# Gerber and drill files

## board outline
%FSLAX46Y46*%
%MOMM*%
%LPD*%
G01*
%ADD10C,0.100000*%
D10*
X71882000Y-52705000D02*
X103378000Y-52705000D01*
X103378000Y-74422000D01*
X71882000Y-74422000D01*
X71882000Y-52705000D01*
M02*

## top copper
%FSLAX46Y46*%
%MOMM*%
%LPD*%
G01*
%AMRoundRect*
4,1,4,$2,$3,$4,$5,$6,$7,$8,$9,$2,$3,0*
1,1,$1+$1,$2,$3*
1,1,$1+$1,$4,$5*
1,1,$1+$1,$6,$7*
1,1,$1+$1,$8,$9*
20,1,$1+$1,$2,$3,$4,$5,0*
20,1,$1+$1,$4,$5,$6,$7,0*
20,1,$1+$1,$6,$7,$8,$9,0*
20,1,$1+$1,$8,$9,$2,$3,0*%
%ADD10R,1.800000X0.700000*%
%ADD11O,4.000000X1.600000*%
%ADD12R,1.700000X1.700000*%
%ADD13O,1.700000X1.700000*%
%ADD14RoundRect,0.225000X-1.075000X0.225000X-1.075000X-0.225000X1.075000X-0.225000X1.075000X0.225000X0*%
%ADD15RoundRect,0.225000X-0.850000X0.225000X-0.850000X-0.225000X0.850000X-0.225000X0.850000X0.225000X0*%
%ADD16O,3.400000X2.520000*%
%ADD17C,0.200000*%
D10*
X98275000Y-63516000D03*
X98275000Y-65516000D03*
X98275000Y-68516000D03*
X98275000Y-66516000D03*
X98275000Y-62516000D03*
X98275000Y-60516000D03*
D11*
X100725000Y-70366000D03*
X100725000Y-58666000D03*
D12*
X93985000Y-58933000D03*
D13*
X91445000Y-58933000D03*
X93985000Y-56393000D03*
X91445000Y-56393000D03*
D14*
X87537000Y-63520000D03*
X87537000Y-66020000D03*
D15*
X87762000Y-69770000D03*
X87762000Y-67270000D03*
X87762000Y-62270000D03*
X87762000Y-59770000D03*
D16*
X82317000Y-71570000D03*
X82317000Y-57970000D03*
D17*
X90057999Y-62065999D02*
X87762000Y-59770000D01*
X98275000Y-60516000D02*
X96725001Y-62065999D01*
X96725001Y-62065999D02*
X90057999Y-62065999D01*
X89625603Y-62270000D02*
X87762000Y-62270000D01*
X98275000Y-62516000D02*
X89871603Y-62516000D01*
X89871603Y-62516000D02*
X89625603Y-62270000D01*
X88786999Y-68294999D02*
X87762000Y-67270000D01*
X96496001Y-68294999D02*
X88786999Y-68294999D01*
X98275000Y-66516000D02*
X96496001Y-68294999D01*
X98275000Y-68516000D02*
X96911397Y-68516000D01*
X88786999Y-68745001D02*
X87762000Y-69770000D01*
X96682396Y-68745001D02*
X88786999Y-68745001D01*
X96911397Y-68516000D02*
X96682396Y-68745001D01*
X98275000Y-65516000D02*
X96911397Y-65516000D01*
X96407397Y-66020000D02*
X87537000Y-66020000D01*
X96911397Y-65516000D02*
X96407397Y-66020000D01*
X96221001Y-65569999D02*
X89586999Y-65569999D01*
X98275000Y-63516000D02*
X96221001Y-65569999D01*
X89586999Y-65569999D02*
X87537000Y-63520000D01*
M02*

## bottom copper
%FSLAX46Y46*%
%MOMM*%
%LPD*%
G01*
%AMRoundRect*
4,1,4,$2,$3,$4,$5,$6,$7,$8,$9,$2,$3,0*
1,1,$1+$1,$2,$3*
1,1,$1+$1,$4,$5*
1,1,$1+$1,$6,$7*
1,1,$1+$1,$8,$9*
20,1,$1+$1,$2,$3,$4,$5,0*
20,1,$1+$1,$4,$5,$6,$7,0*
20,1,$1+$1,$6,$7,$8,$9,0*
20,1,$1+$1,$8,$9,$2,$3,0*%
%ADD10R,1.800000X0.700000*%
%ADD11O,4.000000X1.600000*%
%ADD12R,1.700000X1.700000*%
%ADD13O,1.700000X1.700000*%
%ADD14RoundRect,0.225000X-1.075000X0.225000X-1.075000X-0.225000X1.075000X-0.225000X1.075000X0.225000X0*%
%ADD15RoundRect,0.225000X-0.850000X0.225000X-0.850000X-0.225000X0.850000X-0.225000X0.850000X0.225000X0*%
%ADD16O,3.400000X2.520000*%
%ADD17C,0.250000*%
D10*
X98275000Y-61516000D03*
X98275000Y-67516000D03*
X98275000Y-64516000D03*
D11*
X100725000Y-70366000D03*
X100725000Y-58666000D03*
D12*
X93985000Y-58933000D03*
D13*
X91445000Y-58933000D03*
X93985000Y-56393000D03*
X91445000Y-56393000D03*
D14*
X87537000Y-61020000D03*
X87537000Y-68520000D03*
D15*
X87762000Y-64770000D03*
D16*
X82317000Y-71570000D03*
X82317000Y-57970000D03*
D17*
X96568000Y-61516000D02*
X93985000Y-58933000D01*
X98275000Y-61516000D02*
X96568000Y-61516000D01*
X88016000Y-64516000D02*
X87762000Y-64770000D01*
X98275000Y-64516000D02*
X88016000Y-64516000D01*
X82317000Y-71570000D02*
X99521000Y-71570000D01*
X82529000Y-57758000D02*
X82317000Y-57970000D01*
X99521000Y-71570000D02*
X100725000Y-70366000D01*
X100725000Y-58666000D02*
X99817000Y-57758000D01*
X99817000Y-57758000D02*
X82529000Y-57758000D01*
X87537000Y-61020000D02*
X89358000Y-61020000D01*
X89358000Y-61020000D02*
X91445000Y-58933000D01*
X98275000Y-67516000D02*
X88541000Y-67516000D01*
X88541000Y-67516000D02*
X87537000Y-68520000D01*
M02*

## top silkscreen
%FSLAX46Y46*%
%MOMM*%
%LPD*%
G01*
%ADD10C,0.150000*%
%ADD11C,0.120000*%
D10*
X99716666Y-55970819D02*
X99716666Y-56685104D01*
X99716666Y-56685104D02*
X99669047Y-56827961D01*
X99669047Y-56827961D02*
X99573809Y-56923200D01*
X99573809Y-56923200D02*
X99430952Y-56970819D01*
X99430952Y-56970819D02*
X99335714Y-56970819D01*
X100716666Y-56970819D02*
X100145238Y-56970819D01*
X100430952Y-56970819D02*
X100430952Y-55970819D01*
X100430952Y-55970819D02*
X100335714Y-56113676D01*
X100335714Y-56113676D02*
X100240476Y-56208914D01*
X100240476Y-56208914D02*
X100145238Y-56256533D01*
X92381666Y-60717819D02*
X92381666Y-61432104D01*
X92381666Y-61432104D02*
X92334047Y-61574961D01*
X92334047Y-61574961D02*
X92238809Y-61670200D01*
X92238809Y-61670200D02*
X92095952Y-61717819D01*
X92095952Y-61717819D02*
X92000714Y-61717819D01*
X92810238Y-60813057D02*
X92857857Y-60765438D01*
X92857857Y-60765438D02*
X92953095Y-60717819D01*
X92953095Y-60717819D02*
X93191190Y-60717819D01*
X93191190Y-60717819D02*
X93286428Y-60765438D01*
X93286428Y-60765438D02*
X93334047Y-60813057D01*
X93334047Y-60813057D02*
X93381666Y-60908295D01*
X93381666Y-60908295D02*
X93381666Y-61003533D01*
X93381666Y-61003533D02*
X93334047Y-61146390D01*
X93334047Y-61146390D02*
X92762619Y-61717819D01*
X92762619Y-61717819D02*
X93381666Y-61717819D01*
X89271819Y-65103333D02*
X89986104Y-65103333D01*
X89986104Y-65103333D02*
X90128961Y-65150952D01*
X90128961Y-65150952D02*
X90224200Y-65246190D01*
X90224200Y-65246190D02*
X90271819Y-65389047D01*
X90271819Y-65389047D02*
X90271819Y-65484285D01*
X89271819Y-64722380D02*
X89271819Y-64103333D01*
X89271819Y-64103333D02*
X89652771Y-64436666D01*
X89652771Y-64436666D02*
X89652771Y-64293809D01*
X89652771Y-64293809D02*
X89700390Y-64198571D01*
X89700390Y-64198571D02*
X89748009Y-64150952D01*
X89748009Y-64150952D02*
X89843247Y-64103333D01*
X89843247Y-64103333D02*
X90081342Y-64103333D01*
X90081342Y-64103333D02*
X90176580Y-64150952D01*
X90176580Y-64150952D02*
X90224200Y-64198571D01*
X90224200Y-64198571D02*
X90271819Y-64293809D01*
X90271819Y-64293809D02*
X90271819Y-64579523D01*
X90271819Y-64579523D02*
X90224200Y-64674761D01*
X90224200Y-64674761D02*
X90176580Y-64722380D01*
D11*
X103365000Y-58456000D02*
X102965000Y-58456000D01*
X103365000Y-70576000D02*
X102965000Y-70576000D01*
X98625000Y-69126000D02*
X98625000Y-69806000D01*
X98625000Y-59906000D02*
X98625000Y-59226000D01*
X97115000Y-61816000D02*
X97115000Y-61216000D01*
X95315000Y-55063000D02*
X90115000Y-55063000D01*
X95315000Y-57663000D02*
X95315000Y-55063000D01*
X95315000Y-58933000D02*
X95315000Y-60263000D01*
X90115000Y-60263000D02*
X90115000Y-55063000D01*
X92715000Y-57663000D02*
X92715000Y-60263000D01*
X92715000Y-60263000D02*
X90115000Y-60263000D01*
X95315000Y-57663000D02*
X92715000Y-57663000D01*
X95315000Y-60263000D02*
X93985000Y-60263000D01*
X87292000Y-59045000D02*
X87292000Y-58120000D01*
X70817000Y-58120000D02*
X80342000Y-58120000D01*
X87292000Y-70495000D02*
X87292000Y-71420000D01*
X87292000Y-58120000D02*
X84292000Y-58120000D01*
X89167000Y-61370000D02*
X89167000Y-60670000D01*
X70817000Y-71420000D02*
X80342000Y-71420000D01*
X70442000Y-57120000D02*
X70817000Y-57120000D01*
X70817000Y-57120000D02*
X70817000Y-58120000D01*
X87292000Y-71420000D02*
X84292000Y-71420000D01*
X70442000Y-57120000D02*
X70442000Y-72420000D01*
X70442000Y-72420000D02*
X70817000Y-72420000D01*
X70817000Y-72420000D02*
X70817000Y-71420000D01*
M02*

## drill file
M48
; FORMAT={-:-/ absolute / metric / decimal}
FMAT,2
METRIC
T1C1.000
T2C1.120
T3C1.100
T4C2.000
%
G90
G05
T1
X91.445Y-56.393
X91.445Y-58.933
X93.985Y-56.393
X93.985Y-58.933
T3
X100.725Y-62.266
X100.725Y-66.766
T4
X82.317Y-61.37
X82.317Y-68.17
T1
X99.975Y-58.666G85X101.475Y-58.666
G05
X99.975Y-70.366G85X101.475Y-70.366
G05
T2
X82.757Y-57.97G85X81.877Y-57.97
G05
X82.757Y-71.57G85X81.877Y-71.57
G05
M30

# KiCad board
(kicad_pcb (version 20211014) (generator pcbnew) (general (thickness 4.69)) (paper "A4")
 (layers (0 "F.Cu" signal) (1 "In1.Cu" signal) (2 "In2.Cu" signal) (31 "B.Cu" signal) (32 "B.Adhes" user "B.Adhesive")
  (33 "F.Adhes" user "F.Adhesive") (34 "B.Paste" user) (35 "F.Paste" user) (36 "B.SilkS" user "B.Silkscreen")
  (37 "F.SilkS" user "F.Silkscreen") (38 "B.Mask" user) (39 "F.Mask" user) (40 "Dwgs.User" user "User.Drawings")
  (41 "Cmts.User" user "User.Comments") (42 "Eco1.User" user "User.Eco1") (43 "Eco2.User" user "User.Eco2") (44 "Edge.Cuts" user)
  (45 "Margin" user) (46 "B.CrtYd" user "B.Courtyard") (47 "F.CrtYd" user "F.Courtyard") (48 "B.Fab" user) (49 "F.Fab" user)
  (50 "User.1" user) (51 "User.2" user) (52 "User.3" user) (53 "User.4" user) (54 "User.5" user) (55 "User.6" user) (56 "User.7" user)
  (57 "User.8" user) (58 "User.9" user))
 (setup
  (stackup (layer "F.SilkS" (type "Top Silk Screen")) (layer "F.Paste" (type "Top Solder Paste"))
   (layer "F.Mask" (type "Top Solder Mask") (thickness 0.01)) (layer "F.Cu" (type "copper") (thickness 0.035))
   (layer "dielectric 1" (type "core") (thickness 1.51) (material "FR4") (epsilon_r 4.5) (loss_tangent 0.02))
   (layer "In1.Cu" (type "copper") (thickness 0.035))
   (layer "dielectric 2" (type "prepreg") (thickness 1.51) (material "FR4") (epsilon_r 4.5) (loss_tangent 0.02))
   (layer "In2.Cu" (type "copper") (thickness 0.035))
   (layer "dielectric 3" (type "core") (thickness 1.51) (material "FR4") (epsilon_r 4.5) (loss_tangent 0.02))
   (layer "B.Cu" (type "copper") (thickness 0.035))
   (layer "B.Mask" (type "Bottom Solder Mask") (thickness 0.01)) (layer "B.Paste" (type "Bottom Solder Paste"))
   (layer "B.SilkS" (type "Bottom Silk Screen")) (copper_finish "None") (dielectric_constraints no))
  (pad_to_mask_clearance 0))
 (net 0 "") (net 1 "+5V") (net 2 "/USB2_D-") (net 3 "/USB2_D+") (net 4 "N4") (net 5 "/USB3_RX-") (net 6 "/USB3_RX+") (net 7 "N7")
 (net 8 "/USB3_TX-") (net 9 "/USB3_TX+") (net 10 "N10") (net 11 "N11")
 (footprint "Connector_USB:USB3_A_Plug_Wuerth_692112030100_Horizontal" (layer "F.Cu") (at 100.05 64.516)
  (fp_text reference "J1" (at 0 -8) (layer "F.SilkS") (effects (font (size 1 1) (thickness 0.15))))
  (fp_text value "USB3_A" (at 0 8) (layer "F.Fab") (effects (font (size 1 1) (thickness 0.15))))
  (fp_line (start 3.315 -6.06) (end 2.915 -6.06) (layer "F.SilkS") (width 0.12))
  (fp_line (start 3.315 6.06) (end 2.915 6.06) (layer "F.SilkS") (width 0.12))
  (fp_line (start -1.425 4.61) (end -1.425 5.29) (layer "F.SilkS") (width 0.12))
  (fp_line (start -1.425 -4.61) (end -1.425 -5.29) (layer "F.SilkS") (width 0.12))
  (fp_line (start -2.935 -2.7) (end -2.935 -3.3) (layer "F.SilkS") (width 0.12))
  (pad "" np_thru_hole circle (at 0.675 2.25 90) (size 1.1 1.1) (drill 1.1) (layers *.Cu *.Mask))
  (pad "" np_thru_hole circle (at 0.675 -2.25 90) (size 1.1 1.1) (drill 1.1) (layers *.Cu *.Mask))
  (pad "1" smd rect (at -1.775 -3 90) (size 0.7 1.8) (layers "B.Cu" "F.Paste" "F.Mask") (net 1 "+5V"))
  (pad "2" smd rect (at -1.775 -1 90) (size 0.7 1.8) (layers "F.Cu" "F.Paste" "F.Mask") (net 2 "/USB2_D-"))
  (pad "3" smd rect (at -1.775 1 90) (size 0.7 1.8) (layers "F.Cu" "F.Paste" "F.Mask") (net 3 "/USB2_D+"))
  (pad "4" smd rect (at -1.775 3 90) (size 0.7 1.8) (layers "B.Cu" "F.Paste" "F.Mask") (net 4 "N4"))
  (pad "5" smd rect (at -1.775 4 90) (size 0.7 1.8) (layers "F.Cu" "F.Paste" "F.Mask") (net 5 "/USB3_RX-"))
  (pad "6" smd rect (at -1.775 2 90) (size 0.7 1.8) (layers "F.Cu" "F.Paste" "F.Mask") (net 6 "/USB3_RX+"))
  (pad "7" smd rect (at -1.775 0 90) (size 0.7 1.8) (layers "B.Cu" "F.Paste" "F.Mask") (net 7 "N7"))
  (pad "8" smd rect (at -1.775 -2 90) (size 0.7 1.8) (layers "F.Cu" "F.Paste" "F.Mask") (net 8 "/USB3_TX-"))
  (pad "9" smd rect (at -1.775 -4) (size 1.8 0.7) (layers "F.Cu" "F.Paste" "F.Mask") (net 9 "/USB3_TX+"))
  (pad "10" thru_hole oval (at 0.675 5.85 90) (size 1.6 4) (drill oval 1 2.5) (layers *.Cu *.Mask) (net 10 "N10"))
  (pad "10" thru_hole oval (at 0.675 -5.85 90) (size 1.6 4) (drill oval 1 2.5) (layers *.Cu *.Mask) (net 10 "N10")))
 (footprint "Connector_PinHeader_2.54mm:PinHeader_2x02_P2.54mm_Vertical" (layer "F.Cu") (at 93.985 58.933 180)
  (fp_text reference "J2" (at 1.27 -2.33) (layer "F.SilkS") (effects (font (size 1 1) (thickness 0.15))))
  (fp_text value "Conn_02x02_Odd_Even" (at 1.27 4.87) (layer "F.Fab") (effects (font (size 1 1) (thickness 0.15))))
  (fp_line (start -1.33 3.87) (end 3.87 3.87) (layer "F.SilkS") (width 0.12))
  (fp_line (start -1.33 1.27) (end -1.33 3.87) (layer "F.SilkS") (width 0.12))
  (fp_line (start -1.33 0) (end -1.33 -1.33) (layer "F.SilkS") (width 0.12))
  (fp_line (start 3.87 -1.33) (end 3.87 3.87) (layer "F.SilkS") (width 0.12))
  (fp_line (start 1.27 1.27) (end 1.27 -1.33) (layer "F.SilkS") (width 0.12))
  (fp_line (start 1.27 -1.33) (end 3.87 -1.33) (layer "F.SilkS") (width 0.12))
  (fp_line (start -1.33 1.27) (end 1.27 1.27) (layer "F.SilkS") (width 0.12))
  (fp_line (start -1.33 -1.33) (end 0 -1.33) (layer "F.SilkS") (width 0.12))
  (pad "1" thru_hole rect (at 0 0 180) (size 1.7 1.7) (drill 1) (layers *.Cu *.Mask) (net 1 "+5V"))
  (pad "2" thru_hole oval (at 2.54 0 180) (size 1.7 1.7) (drill 1) (layers *.Cu *.Mask) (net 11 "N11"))
  (pad "3" thru_hole oval (at 0 2.54 180) (size 1.7 1.7) (drill 1) (layers *.Cu *.Mask) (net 1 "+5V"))
  (pad "4" thru_hole oval (at 2.54 2.54 180) (size 1.7 1.7) (drill 1) (layers *.Cu *.Mask) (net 11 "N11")))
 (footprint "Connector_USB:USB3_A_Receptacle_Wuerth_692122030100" (layer "F.Cu") (at 78.867 64.77 -90)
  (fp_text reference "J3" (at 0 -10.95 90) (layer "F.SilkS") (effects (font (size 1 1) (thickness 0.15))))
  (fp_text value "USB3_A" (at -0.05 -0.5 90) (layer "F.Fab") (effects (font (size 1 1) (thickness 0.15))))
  (fp_line (start -5.725 -8.425) (end -6.65 -8.425) (layer "F.SilkS") (width 0.12))
  (fp_line (start -6.65 8.05) (end -6.65 -1.475) (layer "F.SilkS") (width 0.12))
  (fp_line (start 5.725 -8.425) (end 6.65 -8.425) (layer "F.SilkS") (width 0.12))
  (fp_line (start -6.65 -8.425) (end -6.65 -5.425) (layer "F.SilkS") (width 0.12))
  (fp_line (start -3.4 -10.3) (end -4.1 -10.3) (layer "F.SilkS") (width 0.12))
  (fp_line (start 6.65 8.05) (end 6.65 -1.475) (layer "F.SilkS") (width 0.12))
  (fp_line (start -7.65 8.425) (end -7.65 8.05) (layer "F.SilkS") (width 0.12))
  (fp_line (start -7.65 8.05) (end -6.65 8.05) (layer "F.SilkS") (width 0.12))
  (fp_line (start 6.65 -8.425) (end 6.65 -5.425) (layer "F.SilkS") (width 0.12))
  (fp_line (start -7.65 8.425) (end 7.65 8.425) (layer "F.SilkS") (width 0.12))
  (fp_line (start 7.65 8.425) (end 7.65 8.05) (layer "F.SilkS") (width 0.12))
  (fp_line (start 7.65 8.05) (end 6.65 8.05) (layer "F.SilkS") (width 0.12))
  (pad "" np_thru_hole circle (at 3.4 -3.45 270) (size 2 2) (drill 2) (layers F&B.Cu *.Mask))
  (pad "" np_thru_hole circle (at -3.4 -3.45 270) (size 2 2) (drill 2) (layers F&B.Cu *.Mask))
  (pad "1" smd roundrect (at -3.75 -8.67 270) (size 0.9 2.6) (layers "B.Cu" "F.Paste" "F.Mask") (roundrect_rratio 0.25) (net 11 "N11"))
  (pad "2" smd roundrect (at -1.25 -8.67 270) (size 0.9 2.6) (layers "F.Cu" "F.Paste" "F.Mask") (roundrect_rratio 0.25) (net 2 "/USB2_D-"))
  (pad "3" smd roundrect (at 1.25 -8.67 270) (size 0.9 2.6) (layers "F.Cu" "F.Paste" "F.Mask") (roundrect_rratio 0.25) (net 3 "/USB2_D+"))
  (pad "4" smd roundrect (at 3.75 -8.67 270) (size 0.9 2.6) (layers "B.Cu" "F.Paste" "F.Mask") (roundrect_rratio 0.25) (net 4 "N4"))
  (pad "5" smd roundrect (at 5 -8.895 270) (size 0.9 2.15) (layers "F.Cu" "F.Paste" "F.Mask") (roundrect_rratio 0.25) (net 5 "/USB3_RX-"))
  (pad "6" smd roundrect (at 2.5 -8.895 270) (size 0.9 2.15) (layers "F.Cu" "F.Paste" "F.Mask") (roundrect_rratio 0.25) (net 6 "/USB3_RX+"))
  (pad "7" smd roundrect (at 0 -8.895 270) (size 0.9 2.15) (layers "B.Cu" "F.Paste" "F.Mask") (roundrect_rratio 0.25) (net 7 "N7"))
  (pad "8" smd roundrect (at -2.5 -8.895 270) (size 0.9 2.15) (layers "F.Cu" "F.Paste" "F.Mask") (roundrect_rratio 0.25) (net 8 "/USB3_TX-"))
  (pad "9" smd roundrect (at -5 -8.895 270) (size 0.9 2.15) (layers "F.Cu" "F.Paste" "F.Mask") (roundrect_rratio 0.25) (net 9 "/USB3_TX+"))
  (pad "10" thru_hole oval (at 6.8 -3.45 270) (size 2.52 3.4) (drill oval 1.12 2) (layers *.Cu *.Mask) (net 10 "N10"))
  (pad "10" thru_hole oval (at -6.8 -3.45 270) (size 2.52 3.4) (drill oval 1.12 2) (layers *.Cu *.Mask) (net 10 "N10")))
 (gr_rect (start 103.378 52.705) (end 71.882 74.422) (layer "Edge.Cuts") (width 0.1) (fill none))
 (segment (start 96.568 61.516) (end 93.985 58.933) (width 0.25) (layer "B.Cu") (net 1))
 (segment (start 98.275 61.516) (end 96.568 61.516) (width 0.25) (layer "B.Cu") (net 1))
 (segment (start 90.057999 62.065999) (end 87.762 59.77) (width 0.2) (layer "F.Cu") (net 9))
 (segment (start 98.275 60.516) (end 96.725001 62.065999) (width 0.2) (layer "F.Cu") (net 9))
 (segment (start 96.725001 62.065999) (end 90.057999 62.065999) (width 0.2) (layer "F.Cu") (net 9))
 (segment (start 89.625603 62.27) (end 87.762 62.27) (width 0.2) (layer "F.Cu") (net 8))
 (segment (start 98.275 62.516) (end 89.871603 62.516) (width 0.2) (layer "F.Cu") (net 8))
 (segment (start 89.871603 62.516) (end 89.625603 62.27) (width 0.2) (layer "F.Cu") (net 8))
 (segment (start 88.786999 68.294999) (end 87.762 67.27) (width 0.2) (layer "F.Cu") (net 6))
 (segment (start 96.496001 68.294999) (end 88.786999 68.294999) (width 0.2) (layer "F.Cu") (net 6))
 (segment (start 98.275 66.516) (end 96.496001 68.294999) (width 0.2) (layer "F.Cu") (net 6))
 (segment (start 98.275 68.516) (end 96.911397 68.516) (width 0.2) (layer "F.Cu") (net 5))
 (segment (start 88.786999 68.745001) (end 87.762 69.77) (width 0.2) (layer "F.Cu") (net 5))
 (segment (start 96.682396 68.745001) (end 88.786999 68.745001) (width 0.2) (layer "F.Cu") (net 5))
 (segment (start 96.911397 68.516) (end 96.682396 68.745001) (width 0.2) (layer "F.Cu") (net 5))
 (segment (start 88.016 64.516) (end 87.762 64.77) (width 0.25) (layer "B.Cu") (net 7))
 (segment (start 98.275 64.516) (end 88.016 64.516) (width 0.25) (layer "B.Cu") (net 7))
 (segment (start 98.275 65.516) (end 96.911397 65.516) (width 0.2) (layer "F.Cu") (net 3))
 (segment (start 96.407397 66.02) (end 87.537 66.02) (width 0.2) (layer "F.Cu") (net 3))
 (segment (start 96.911397 65.516) (end 96.407397 66.02) (width 0.2) (layer "F.Cu") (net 3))
 (segment (start 96.221001 65.569999) (end 89.586999 65.569999) (width 0.2) (layer "F.Cu") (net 2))
 (segment (start 98.275 63.516) (end 96.221001 65.569999) (width 0.2) (layer "F.Cu") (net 2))
 (segment (start 89.586999 65.569999) (end 87.537 63.52) (width 0.2) (layer "F.Cu") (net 2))
 (segment (start 82.317 71.57) (end 99.521 71.57) (width 0.25) (layer "B.Cu") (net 10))
 (segment (start 82.529 57.758) (end 82.317 57.97) (width 0.25) (layer "B.Cu") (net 10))
 (segment (start 99.521 71.57) (end 100.725 70.366) (width 0.25) (layer "B.Cu") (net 10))
 (segment (start 100.725 58.666) (end 99.817 57.758) (width 0.25) (layer "B.Cu") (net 10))
 (segment (start 99.817 57.758) (end 82.529 57.758) (width 0.25) (layer "B.Cu") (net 10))
 (segment (start 87.537 61.02) (end 89.358 61.02) (width 0.25) (layer "B.Cu") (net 11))
 (segment (start 89.358 61.02) (end 91.445 58.933) (width 0.25) (layer "B.Cu") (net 11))
 (segment (start 98.275 67.516) (end 88.541 67.516) (width 0.25) (layer "B.Cu") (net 4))
 (segment (start 88.541 67.516) (end 87.537 68.52) (width 0.25) (layer "B.Cu") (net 4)))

